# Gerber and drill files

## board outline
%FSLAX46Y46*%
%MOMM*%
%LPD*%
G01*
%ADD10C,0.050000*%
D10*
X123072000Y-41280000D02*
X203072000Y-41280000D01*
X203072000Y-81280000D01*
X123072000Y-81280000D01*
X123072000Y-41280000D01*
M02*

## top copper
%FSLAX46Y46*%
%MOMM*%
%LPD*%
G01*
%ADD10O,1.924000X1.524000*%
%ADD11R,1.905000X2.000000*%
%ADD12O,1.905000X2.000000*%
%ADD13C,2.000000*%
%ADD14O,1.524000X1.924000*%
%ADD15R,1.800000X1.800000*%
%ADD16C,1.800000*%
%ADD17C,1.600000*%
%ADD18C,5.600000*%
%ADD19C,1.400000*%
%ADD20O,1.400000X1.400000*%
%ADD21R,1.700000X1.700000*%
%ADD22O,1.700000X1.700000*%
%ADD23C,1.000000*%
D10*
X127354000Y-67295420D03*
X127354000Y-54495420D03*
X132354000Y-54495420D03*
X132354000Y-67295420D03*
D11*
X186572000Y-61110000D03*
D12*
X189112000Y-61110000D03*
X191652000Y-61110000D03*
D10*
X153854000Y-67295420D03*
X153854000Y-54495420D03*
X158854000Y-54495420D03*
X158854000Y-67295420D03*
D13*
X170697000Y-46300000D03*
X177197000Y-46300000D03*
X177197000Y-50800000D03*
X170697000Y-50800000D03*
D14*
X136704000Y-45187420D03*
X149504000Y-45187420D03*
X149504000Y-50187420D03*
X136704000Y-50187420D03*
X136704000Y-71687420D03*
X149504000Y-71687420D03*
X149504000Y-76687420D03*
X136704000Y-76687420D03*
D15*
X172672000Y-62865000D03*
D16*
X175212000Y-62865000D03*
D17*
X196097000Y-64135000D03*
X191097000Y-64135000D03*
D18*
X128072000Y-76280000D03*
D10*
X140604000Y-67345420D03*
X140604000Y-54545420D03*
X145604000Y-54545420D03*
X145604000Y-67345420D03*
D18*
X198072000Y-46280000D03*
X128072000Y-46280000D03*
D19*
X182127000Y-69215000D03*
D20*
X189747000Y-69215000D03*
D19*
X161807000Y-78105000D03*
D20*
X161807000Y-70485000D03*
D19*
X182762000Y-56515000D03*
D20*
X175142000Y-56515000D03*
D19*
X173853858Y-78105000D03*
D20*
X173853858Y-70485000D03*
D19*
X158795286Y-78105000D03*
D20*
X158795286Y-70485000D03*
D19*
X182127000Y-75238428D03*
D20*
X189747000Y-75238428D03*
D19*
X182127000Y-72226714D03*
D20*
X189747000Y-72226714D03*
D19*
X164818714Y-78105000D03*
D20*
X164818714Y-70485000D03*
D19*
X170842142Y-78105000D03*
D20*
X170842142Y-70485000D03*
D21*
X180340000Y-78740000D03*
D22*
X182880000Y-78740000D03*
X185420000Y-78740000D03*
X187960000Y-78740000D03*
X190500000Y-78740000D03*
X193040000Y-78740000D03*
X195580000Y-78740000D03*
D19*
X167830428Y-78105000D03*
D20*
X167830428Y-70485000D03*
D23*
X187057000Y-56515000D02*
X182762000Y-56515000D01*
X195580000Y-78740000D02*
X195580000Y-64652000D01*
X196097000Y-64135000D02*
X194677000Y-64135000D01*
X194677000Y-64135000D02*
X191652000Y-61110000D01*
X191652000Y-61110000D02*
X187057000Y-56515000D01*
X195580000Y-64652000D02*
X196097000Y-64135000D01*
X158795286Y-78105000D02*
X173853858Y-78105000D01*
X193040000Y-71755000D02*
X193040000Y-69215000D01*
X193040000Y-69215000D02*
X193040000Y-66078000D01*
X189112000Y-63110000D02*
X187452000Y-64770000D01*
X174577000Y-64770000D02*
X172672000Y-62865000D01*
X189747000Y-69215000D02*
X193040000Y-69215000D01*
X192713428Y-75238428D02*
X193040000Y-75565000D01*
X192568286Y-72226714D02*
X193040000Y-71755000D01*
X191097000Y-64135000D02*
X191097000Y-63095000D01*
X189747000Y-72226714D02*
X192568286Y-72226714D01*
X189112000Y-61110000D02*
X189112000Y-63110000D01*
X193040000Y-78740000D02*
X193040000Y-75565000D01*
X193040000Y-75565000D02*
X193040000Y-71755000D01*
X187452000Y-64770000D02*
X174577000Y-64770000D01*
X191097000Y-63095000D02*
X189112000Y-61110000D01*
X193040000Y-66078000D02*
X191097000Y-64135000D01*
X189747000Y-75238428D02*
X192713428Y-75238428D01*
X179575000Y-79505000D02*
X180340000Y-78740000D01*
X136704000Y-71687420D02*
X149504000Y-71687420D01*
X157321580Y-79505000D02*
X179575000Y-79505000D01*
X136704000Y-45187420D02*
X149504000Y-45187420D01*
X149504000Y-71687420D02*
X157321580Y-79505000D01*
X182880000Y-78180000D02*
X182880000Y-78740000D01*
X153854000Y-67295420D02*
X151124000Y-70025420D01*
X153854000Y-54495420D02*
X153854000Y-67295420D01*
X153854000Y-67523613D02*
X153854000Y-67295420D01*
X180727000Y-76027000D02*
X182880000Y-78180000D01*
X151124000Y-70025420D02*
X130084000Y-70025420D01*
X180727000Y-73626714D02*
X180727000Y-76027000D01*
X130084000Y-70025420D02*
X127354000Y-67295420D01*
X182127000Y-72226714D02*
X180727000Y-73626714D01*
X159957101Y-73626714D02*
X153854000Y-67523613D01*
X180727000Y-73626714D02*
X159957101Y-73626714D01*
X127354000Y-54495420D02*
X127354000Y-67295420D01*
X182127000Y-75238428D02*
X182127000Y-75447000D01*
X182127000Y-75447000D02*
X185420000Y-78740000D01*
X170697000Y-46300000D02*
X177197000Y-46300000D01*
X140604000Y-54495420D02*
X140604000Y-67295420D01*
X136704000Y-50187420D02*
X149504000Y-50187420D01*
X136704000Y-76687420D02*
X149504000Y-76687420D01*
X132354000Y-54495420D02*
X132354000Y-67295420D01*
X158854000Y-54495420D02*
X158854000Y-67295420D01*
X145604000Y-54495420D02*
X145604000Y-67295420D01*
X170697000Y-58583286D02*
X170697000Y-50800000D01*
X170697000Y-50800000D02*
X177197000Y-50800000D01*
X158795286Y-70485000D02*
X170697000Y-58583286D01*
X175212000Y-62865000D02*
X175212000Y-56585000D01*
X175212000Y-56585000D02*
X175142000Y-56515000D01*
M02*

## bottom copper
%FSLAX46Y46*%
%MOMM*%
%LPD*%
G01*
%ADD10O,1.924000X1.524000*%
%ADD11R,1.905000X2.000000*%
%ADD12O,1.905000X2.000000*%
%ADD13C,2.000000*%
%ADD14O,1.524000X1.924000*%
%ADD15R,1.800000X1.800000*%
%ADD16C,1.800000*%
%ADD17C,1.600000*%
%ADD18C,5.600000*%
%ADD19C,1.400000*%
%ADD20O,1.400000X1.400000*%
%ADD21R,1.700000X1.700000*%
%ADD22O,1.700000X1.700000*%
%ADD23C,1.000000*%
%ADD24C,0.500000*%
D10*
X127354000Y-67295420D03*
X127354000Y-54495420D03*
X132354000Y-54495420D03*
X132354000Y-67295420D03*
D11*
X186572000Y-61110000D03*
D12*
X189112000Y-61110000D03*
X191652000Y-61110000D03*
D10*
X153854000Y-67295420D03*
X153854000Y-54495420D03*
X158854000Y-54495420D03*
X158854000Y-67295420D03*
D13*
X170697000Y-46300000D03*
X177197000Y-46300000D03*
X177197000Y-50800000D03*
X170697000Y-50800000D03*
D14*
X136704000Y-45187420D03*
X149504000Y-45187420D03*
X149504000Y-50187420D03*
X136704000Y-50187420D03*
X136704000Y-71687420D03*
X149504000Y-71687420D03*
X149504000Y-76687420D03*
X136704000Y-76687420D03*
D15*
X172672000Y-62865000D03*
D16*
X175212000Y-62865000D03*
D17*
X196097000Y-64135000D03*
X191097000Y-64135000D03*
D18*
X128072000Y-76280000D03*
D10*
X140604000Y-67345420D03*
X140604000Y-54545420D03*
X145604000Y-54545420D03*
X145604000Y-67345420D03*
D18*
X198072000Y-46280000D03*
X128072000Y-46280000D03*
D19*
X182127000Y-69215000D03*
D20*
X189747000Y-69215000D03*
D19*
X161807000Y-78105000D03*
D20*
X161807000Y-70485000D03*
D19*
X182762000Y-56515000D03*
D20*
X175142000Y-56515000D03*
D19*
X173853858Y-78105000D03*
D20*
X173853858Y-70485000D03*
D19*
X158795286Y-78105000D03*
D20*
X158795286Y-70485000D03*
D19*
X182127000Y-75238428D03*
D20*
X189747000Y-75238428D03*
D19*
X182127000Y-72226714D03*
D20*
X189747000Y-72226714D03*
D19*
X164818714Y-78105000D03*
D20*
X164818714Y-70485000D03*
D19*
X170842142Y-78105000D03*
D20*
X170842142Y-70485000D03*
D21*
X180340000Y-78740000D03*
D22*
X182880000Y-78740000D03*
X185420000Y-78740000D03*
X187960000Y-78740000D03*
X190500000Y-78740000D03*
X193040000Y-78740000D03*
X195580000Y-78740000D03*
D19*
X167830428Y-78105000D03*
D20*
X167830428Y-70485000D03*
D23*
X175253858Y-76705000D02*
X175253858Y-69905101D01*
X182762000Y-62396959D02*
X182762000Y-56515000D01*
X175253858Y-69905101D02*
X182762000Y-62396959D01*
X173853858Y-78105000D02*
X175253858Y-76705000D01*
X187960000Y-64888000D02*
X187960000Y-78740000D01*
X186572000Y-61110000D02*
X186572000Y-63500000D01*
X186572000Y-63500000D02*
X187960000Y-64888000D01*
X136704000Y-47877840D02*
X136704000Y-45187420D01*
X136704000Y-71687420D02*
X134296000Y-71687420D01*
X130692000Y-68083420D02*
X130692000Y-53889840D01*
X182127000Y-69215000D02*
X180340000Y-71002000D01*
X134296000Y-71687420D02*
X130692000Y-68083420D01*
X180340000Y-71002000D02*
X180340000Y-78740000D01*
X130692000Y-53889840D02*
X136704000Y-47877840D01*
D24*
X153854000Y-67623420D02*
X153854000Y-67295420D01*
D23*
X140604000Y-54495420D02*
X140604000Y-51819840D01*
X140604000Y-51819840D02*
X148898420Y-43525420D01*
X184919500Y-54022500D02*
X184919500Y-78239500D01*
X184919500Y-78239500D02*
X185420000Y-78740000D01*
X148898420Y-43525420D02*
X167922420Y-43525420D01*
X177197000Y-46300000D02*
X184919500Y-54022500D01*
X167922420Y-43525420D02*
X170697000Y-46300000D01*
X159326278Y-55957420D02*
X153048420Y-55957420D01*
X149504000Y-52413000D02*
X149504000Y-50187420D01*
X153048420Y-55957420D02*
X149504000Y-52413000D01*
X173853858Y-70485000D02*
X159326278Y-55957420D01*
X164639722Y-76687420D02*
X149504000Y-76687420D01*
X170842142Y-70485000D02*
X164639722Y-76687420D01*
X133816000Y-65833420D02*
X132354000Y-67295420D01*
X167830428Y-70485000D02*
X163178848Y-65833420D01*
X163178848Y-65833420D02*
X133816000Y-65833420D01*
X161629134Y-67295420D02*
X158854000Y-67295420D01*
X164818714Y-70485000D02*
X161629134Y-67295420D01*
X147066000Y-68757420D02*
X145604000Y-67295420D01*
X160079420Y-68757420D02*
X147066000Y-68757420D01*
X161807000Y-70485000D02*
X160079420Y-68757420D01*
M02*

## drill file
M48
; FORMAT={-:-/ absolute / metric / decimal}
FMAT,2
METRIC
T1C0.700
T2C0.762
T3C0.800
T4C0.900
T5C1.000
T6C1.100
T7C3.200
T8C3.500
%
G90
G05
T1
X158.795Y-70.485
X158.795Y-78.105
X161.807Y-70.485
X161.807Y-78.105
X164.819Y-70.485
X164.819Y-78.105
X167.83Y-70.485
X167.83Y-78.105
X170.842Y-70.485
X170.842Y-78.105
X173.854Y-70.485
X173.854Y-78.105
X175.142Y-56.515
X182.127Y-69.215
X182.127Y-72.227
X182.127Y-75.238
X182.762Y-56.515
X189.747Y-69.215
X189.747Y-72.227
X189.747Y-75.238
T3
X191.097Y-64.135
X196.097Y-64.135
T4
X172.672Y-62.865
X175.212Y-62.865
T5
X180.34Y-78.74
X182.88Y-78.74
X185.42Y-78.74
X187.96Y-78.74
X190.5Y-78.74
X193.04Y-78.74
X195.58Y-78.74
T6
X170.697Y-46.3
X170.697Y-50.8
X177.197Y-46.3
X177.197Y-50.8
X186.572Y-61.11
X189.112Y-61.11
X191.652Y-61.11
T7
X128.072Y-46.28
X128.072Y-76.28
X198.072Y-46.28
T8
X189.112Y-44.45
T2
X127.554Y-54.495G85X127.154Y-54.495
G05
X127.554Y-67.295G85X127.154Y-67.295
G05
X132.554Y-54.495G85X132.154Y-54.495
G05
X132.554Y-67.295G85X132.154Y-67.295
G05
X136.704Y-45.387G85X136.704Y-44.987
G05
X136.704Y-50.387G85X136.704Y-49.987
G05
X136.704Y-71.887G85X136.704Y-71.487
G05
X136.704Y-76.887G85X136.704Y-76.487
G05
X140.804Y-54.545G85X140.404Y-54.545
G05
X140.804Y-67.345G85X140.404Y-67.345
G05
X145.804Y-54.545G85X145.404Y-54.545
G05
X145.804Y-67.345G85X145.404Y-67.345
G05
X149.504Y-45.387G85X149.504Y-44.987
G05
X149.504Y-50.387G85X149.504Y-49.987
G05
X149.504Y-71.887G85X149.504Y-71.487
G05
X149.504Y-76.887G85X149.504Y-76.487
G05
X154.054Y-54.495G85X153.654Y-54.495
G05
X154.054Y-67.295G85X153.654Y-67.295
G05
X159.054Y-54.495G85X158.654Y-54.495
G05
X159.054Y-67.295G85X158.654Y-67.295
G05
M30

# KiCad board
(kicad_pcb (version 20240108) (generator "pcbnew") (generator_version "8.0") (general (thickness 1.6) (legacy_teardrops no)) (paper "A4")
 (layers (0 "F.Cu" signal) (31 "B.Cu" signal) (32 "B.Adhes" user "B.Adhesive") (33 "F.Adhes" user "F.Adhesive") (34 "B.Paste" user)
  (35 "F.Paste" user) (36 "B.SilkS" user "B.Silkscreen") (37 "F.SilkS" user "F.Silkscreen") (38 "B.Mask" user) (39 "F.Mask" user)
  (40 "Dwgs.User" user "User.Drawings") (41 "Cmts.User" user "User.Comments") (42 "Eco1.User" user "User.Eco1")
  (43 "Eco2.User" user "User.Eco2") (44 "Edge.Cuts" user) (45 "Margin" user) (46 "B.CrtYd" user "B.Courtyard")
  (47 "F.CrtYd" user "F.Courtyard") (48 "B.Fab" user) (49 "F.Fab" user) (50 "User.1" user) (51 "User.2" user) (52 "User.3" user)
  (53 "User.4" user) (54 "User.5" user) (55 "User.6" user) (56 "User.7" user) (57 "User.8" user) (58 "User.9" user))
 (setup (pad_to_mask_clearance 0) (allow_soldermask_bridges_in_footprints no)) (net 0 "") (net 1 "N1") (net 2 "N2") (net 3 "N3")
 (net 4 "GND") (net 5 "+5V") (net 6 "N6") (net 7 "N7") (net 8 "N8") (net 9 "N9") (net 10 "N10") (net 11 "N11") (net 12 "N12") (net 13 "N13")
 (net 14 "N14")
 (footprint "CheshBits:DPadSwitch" (layer "F.Cu") (at 129.854 60.89542 90)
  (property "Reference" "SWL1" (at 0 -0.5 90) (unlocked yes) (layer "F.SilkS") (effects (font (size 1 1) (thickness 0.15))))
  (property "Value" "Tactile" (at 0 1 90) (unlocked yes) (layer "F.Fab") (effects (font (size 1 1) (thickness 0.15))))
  (pad "1" thru_hole oval (at -6.4 -2.5 270) (size 1.524 1.924) (drill oval 0.762 1.162) (layers "*.Cu" "*.Mask") (remove_unused_layers no)
   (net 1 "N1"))
  (pad "2" thru_hole oval (at 6.4 -2.5 270) (size 1.524 1.924) (drill oval 0.762 1.162) (layers "*.Cu" "*.Mask") (remove_unused_layers no)
   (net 1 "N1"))
  (pad "3" thru_hole oval (at 6.4 2.5 270) (size 1.524 1.924) (drill oval 0.762 1.162) (layers "*.Cu" "*.Mask") (remove_unused_layers no)
   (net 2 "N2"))
  (pad "4" thru_hole oval (at -6.4 2.5 270) (size 1.524 1.924) (drill oval 0.762 1.162) (layers "*.Cu" "*.Mask") (remove_unused_layers no)
   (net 2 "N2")))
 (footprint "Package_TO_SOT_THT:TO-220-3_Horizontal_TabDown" (layer "F.Cu") (at 186.572 61.11)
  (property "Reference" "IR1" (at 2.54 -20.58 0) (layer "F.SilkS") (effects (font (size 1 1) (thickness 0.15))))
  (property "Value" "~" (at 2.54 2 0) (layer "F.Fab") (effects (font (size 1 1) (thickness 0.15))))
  (pad "" np_thru_hole circle (at 2.54 -16.66) (size 3.5 3.5) (drill 3.5) (layers "*.Cu" "*.Mask"))
  (pad "1" thru_hole rect (at 0 0) (size 1.905 2) (drill 1.1) (layers "*.Cu" "*.Mask") (remove_unused_layers no) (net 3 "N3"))
  (pad "2" thru_hole oval (at 2.54 0) (size 1.905 2) (drill 1.1) (layers "*.Cu" "*.Mask") (remove_unused_layers no) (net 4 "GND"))
  (pad "3" thru_hole oval (at 5.08 0) (size 1.905 2) (drill 1.1) (layers "*.Cu" "*.Mask") (remove_unused_layers no) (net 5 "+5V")))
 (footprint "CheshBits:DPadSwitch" (layer "F.Cu") (at 156.354 60.89542 90)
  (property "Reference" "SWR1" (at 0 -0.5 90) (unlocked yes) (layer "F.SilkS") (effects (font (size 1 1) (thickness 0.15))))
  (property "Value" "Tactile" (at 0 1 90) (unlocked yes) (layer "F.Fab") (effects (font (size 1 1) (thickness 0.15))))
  (pad "1" thru_hole oval (at -6.4 -2.5 270) (size 1.524 1.924) (drill oval 0.762 1.162) (layers "*.Cu" "*.Mask") (remove_unused_layers no)
   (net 1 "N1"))
  (pad "2" thru_hole oval (at 6.4 -2.5 270) (size 1.524 1.924) (drill oval 0.762 1.162) (layers "*.Cu" "*.Mask") (remove_unused_layers no)
   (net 1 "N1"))
  (pad "3" thru_hole oval (at 6.4 2.5 270) (size 1.524 1.924) (drill oval 0.762 1.162) (layers "*.Cu" "*.Mask") (remove_unused_layers no)
   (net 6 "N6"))
  (pad "4" thru_hole oval (at -6.4 2.5 270) (size 1.524 1.924) (drill oval 0.762 1.162) (layers "*.Cu" "*.Mask") (remove_unused_layers no)
   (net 6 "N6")))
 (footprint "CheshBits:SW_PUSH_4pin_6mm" (layer "F.Cu") (at 170.697 46.3)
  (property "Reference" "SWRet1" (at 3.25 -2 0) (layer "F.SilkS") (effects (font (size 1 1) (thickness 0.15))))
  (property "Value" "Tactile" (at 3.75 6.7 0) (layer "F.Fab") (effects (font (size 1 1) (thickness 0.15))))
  (pad "1" thru_hole circle (at 0 0 90) (size 2 2) (drill 1.1) (layers "*.Cu" "*.Mask") (remove_unused_layers no) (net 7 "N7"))
  (pad "2" thru_hole circle (at 6.5 0 90) (size 2 2) (drill 1.1) (layers "*.Cu" "*.Mask") (remove_unused_layers no) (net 7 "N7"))
  (pad "3" thru_hole circle (at 6.5 4.5 90) (size 2 2) (drill 1.1) (layers "*.Cu" "*.Mask") (remove_unused_layers no) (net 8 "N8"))
  (pad "4" thru_hole circle (at 0 4.5 90) (size 2 2) (drill 1.1) (layers "*.Cu" "*.Mask") (remove_unused_layers no) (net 8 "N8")))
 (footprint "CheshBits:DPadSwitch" (layer "F.Cu") (at 143.104 47.68742)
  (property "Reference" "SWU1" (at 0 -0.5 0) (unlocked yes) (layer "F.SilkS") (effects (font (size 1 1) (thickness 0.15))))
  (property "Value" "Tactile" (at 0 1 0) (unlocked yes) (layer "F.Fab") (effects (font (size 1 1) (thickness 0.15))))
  (pad "1" thru_hole oval (at -6.4 -2.5 180) (size 1.524 1.924) (drill oval 0.762 1.162) (layers "*.Cu" "*.Mask") (remove_unused_layers no)
   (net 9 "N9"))
  (pad "2" thru_hole oval (at 6.4 -2.5 180) (size 1.524 1.924) (drill oval 0.762 1.162) (layers "*.Cu" "*.Mask") (remove_unused_layers no)
   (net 9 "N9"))
  (pad "3" thru_hole oval (at 6.4 2.5 180) (size 1.524 1.924) (drill oval 0.762 1.162) (layers "*.Cu" "*.Mask") (remove_unused_layers no)
   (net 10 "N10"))
  (pad "4" thru_hole oval (at -6.4 2.5 180) (size 1.524 1.924) (drill oval 0.762 1.162) (layers "*.Cu" "*.Mask") (remove_unused_layers no)
   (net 10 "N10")))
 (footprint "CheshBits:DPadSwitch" (layer "F.Cu") (at 143.104 74.18742)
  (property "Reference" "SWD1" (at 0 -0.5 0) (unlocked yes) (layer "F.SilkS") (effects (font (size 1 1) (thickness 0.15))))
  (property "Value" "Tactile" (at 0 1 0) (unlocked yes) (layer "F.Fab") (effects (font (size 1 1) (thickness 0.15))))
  (pad "1" thru_hole oval (at -6.4 -2.5 180) (size 1.524 1.924) (drill oval 0.762 1.162) (layers "*.Cu" "*.Mask") (remove_unused_layers no)
   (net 9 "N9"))
  (pad "2" thru_hole oval (at 6.4 -2.5 180) (size 1.524 1.924) (drill oval 0.762 1.162) (layers "*.Cu" "*.Mask") (remove_unused_layers no)
   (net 9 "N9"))
  (pad "3" thru_hole oval (at 6.4 2.5 180) (size 1.524 1.924) (drill oval 0.762 1.162) (layers "*.Cu" "*.Mask") (remove_unused_layers no)
   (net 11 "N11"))
  (pad "4" thru_hole oval (at -6.4 2.5 180) (size 1.524 1.924) (drill oval 0.762 1.162) (layers "*.Cu" "*.Mask") (remove_unused_layers no)
   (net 11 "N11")))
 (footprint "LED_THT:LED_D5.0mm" (layer "F.Cu") (at 172.672 62.865)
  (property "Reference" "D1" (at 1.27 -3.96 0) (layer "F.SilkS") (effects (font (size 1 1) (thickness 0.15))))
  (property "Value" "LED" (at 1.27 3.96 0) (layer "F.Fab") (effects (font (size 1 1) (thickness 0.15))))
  (pad "1" thru_hole rect (at 0 0) (size 1.8 1.8) (drill 0.9) (layers "*.Cu" "*.Mask") (remove_unused_layers no) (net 4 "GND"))
  (pad "2" thru_hole circle (at 2.54 0) (size 1.8 1.8) (drill 0.9) (layers "*.Cu" "*.Mask") (remove_unused_layers no) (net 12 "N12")))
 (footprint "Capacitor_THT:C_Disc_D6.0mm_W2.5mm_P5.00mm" (layer "F.Cu") (at 196.097 64.135 180)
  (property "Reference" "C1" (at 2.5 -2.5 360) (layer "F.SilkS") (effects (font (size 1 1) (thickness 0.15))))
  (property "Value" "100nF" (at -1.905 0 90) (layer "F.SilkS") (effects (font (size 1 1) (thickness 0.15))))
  (pad "1" thru_hole circle (at 0 0 180) (size 1.6 1.6) (drill 0.8) (layers "*.Cu" "*.Mask") (remove_unused_layers no) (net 5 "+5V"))
  (pad "2" thru_hole circle (at 5 0 180) (size 1.6 1.6) (drill 0.8) (layers "*.Cu" "*.Mask") (remove_unused_layers no) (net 4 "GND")))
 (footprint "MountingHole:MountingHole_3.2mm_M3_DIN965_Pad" (layer "F.Cu") (at 128.072 76.28)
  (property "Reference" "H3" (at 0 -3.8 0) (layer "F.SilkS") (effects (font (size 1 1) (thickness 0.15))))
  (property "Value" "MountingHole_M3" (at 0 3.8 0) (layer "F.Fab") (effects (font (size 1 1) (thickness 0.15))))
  (pad "1" thru_hole circle (at 0 0) (size 5.6 5.6) (drill 3.2) (layers "*.Cu" "*.Mask") (remove_unused_layers no)))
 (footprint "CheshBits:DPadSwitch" (layer "F.Cu") (at 143.104 60.94542 90)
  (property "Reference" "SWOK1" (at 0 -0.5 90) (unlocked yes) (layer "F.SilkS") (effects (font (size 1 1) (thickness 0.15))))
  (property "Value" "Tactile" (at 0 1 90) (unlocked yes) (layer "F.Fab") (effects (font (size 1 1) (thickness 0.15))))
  (pad "1" thru_hole oval (at -6.4 -2.5 270) (size 1.524 1.924) (drill oval 0.762 1.162) (layers "*.Cu" "*.Mask") (remove_unused_layers no)
   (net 7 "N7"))
  (pad "2" thru_hole oval (at 6.4 -2.5 270) (size 1.524 1.924) (drill oval 0.762 1.162) (layers "*.Cu" "*.Mask") (remove_unused_layers no)
   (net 7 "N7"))
  (pad "3" thru_hole oval (at 6.4 2.5 270) (size 1.524 1.924) (drill oval 0.762 1.162) (layers "*.Cu" "*.Mask") (remove_unused_layers no)
   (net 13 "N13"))
  (pad "4" thru_hole oval (at -6.4 2.5 270) (size 1.524 1.924) (drill oval 0.762 1.162) (layers "*.Cu" "*.Mask") (remove_unused_layers no)
   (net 13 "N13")))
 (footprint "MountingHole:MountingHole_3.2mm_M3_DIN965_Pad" (layer "F.Cu") (at 198.072 46.28)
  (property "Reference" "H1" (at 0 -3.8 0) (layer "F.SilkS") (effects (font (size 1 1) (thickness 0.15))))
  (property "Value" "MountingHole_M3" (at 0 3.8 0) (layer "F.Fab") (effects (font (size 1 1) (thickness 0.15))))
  (pad "1" thru_hole circle (at 0 0) (size 5.6 5.6) (drill 3.2) (layers "*.Cu" "*.Mask") (remove_unused_layers no)))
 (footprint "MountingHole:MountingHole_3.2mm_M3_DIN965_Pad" (layer "F.Cu") (at 128.072 46.28)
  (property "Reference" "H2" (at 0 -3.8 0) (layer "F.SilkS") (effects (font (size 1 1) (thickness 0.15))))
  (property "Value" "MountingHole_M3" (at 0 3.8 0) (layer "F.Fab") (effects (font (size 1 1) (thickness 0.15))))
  (pad "1" thru_hole circle (at 0 0) (size 5.6 5.6) (drill 3.2) (layers "*.Cu" "*.Mask") (remove_unused_layers no)))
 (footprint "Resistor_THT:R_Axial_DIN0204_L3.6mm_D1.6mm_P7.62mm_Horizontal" (layer "B.Cu") (at 182.127 69.215)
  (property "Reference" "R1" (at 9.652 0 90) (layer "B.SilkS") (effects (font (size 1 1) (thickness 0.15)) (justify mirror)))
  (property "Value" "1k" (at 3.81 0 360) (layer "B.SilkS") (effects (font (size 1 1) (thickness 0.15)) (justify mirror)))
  (pad "1" thru_hole circle (at 0 0) (size 1.4 1.4) (drill 0.7) (layers "*.Cu" "*.Mask") (remove_unused_layers no) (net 9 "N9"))
  (pad "2" thru_hole oval (at 7.62 0) (size 1.4 1.4) (drill 0.7) (layers "*.Cu" "*.Mask") (remove_unused_layers no) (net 4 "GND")))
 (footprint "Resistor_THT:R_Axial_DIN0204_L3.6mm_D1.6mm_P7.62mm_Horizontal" (layer "B.Cu") (at 161.807 78.105 90)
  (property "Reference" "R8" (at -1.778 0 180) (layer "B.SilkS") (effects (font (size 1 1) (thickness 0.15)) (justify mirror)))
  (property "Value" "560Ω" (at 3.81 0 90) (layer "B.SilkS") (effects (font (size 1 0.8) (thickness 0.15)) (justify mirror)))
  (pad "1" thru_hole circle (at 0 0 90) (size 1.4 1.4) (drill 0.7) (layers "*.Cu" "*.Mask") (remove_unused_layers no) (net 5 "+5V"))
  (pad "2" thru_hole oval (at 7.62 0 90) (size 1.4 1.4) (drill 0.7) (layers "*.Cu" "*.Mask") (remove_unused_layers no) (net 13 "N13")))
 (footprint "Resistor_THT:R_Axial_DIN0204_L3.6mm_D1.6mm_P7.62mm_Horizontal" (layer "B.Cu") (at 182.762 56.515 180)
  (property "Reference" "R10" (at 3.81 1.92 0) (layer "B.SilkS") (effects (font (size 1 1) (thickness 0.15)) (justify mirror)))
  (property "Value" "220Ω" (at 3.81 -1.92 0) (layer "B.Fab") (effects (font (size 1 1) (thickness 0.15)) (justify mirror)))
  (pad "1" thru_hole circle (at 0 0 180) (size 1.4 1.4) (drill 0.7) (layers "*.Cu" "*.Mask") (remove_unused_layers no) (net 5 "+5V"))
  (pad "2" thru_hole oval (at 7.62 0 180) (size 1.4 1.4) (drill 0.7) (layers "*.Cu" "*.Mask") (remove_unused_layers no) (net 12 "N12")))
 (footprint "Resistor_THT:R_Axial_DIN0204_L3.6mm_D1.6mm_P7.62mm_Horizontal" (layer "B.Cu") (at 173.853858 78.105 90)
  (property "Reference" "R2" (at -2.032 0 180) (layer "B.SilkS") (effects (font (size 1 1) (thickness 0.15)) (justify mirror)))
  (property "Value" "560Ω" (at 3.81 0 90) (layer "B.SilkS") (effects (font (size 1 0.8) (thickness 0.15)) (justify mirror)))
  (pad "1" thru_hole circle (at 0 0 90) (size 1.4 1.4) (drill 0.7) (layers "*.Cu" "*.Mask") (remove_unused_layers no) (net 5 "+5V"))
  (pad "2" thru_hole oval (at 7.62 0 90) (size 1.4 1.4) (drill 0.7) (layers "*.Cu" "*.Mask") (remove_unused_layers no) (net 10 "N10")))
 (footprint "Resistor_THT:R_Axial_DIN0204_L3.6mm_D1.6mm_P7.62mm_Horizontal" (layer "B.Cu") (at 158.795286 78.105 90)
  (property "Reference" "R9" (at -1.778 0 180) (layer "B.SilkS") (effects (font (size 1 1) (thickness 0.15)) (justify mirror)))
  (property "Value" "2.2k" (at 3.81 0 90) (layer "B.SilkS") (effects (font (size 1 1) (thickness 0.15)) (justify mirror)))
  (pad "1" thru_hole circle (at 0 0 90) (size 1.4 1.4) (drill 0.7) (layers "*.Cu" "*.Mask") (remove_unused_layers no) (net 5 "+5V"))
  (pad "2" thru_hole oval (at 7.62 0 90) (size 1.4 1.4) (drill 0.7) (layers "*.Cu" "*.Mask") (remove_unused_layers no) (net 8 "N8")))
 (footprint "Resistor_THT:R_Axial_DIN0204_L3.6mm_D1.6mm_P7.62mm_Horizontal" (layer "B.Cu") (at 182.127 75.238428)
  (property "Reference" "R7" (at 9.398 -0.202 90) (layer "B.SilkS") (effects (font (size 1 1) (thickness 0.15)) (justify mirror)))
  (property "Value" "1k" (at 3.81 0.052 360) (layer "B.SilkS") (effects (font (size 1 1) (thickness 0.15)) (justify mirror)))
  (pad "1" thru_hole circle (at 0 0) (size 1.4 1.4) (drill 0.7) (layers "*.Cu" "*.Mask") (remove_unused_layers no) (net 7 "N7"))
  (pad "2" thru_hole oval (at 7.62 0) (size 1.4 1.4) (drill 0.7) (layers "*.Cu" "*.Mask") (remove_unused_layers no) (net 4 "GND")))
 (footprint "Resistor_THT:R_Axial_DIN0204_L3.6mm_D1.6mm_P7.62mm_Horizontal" (layer "B.Cu") (at 182.127 72.226714)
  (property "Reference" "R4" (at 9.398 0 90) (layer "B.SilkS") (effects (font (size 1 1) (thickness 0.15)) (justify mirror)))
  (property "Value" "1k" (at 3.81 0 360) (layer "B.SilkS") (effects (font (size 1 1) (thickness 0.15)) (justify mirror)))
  (pad "1" thru_hole circle (at 0 0) (size 1.4 1.4) (drill 0.7) (layers "*.Cu" "*.Mask") (remove_unused_layers no) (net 1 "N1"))
  (pad "2" thru_hole oval (at 7.62 0) (size 1.4 1.4) (drill 0.7) (layers "*.Cu" "*.Mask") (remove_unused_layers no) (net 4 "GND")))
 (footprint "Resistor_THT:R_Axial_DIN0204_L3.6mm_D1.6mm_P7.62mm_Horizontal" (layer "B.Cu") (at 164.818714 78.105 90)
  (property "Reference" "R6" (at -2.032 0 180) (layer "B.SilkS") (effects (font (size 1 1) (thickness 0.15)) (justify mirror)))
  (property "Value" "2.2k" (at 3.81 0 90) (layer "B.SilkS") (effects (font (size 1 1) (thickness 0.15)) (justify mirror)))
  (pad "1" thru_hole circle (at 0 0 90) (size 1.4 1.4) (drill 0.7) (layers "*.Cu" "*.Mask") (remove_unused_layers no) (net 5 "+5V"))
  (pad "2" thru_hole oval (at 7.62 0 90) (size 1.4 1.4) (drill 0.7) (layers "*.Cu" "*.Mask") (remove_unused_layers no) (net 6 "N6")))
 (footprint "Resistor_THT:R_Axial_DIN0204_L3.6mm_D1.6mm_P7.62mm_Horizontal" (layer "B.Cu") (at 170.842142 78.105 90)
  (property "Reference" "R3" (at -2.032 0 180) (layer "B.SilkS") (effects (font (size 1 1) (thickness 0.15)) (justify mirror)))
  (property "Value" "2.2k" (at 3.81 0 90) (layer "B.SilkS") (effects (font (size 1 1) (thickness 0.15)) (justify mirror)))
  (pad "1" thru_hole circle (at 0 0 90) (size 1.4 1.4) (drill 0.7) (layers "*.Cu" "*.Mask") (remove_unused_layers no) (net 5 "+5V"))
  (pad "2" thru_hole oval (at 7.62 0 90) (size 1.4 1.4) (drill 0.7) (layers "*.Cu" "*.Mask") (remove_unused_layers no) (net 11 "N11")))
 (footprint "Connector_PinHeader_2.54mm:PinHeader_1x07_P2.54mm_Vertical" (layer "B.Cu") (at 180.34 78.74 -90)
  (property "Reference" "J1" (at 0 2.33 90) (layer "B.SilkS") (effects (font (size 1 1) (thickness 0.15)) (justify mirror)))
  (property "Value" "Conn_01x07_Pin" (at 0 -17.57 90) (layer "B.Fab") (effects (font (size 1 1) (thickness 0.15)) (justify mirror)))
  (pad "1" thru_hole rect (at 0 0 270) (size 1.7 1.7) (drill 1) (layers "*.Cu" "*.Mask") (remove_unused_layers no) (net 9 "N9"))
  (pad "2" thru_hole oval (at 0 -2.54 270) (size 1.7 1.7) (drill 1) (layers "*.Cu" "*.Mask") (remove_unused_layers no) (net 1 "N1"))
  (pad "3" thru_hole oval (at 0 -5.08 270) (size 1.7 1.7) (drill 1) (layers "*.Cu" "*.Mask") (remove_unused_layers no) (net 7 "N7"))
  (pad "4" thru_hole oval (at 0 -7.62 270) (size 1.7 1.7) (drill 1) (layers "*.Cu" "*.Mask") (remove_unused_layers no) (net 3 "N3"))
  (pad "5" thru_hole oval (at 0 -10.16 270) (size 1.7 1.7) (drill 1) (layers "*.Cu" "*.Mask") (remove_unused_layers no) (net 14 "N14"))
  (pad "6" thru_hole oval (at 0 -12.7 270) (size 1.7 1.7) (drill 1) (layers "*.Cu" "*.Mask") (remove_unused_layers no) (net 4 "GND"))
  (pad "7" thru_hole oval (at 0 -15.24 270) (size 1.7 1.7) (drill 1) (layers "*.Cu" "*.Mask") (remove_unused_layers no) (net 5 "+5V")))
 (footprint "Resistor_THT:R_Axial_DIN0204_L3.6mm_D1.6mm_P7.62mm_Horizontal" (layer "B.Cu") (at 167.830428 78.105 90)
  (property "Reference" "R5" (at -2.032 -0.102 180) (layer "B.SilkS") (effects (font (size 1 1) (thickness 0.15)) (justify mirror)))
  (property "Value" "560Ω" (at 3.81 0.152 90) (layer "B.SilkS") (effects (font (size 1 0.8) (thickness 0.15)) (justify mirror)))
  (pad "1" thru_hole circle (at 0 0 90) (size 1.4 1.4) (drill 0.7) (layers "*.Cu" "*.Mask") (remove_unused_layers no) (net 5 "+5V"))
  (pad "2" thru_hole oval (at 7.62 0 90) (size 1.4 1.4) (drill 0.7) (layers "*.Cu" "*.Mask") (remove_unused_layers no) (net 2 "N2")))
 (gr_rect (start 123.072 41.28) (end 203.072 81.28) (stroke (width 0.05) (type default)) (fill none) (layer "Edge.Cuts"))
 (segment (start 187.057 56.515) (end 182.762 56.515) (width 1) (layer "F.Cu") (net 5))
 (segment (start 195.58 78.74) (end 195.58 64.652) (width 1) (layer "F.Cu") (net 5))
 (segment (start 196.097 64.135) (end 194.677 64.135) (width 1) (layer "F.Cu") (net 5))
 (segment (start 194.677 64.135) (end 191.652 61.11) (width 1) (layer "F.Cu") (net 5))
 (segment (start 191.652 61.11) (end 187.057 56.515) (width 1) (layer "F.Cu") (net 5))
 (segment (start 195.58 64.652) (end 196.097 64.135) (width 1) (layer "F.Cu") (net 5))
 (segment (start 158.795286 78.105) (end 173.853858 78.105) (width 1) (layer "F.Cu") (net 5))
 (segment (start 175.253858 76.705) (end 175.253858 69.905101) (width 1) (layer "B.Cu") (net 5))
 (segment (start 182.762 62.396959) (end 182.762 56.515) (width 1) (layer "B.Cu") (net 5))
 (segment (start 175.253858 69.905101) (end 182.762 62.396959) (width 1) (layer "B.Cu") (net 5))
 (segment (start 173.853858 78.105) (end 175.253858 76.705) (width 1) (layer "B.Cu") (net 5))
 (segment (start 193.04 71.755) (end 193.04 69.215) (width 1) (layer "F.Cu") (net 4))
 (segment (start 193.04 69.215) (end 193.04 66.078) (width 1) (layer "F.Cu") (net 4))
 (segment (start 189.112 63.11) (end 187.452 64.77) (width 1) (layer "F.Cu") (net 4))
 (segment (start 174.577 64.77) (end 172.672 62.865) (width 1) (layer "F.Cu") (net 4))
 (segment (start 189.747 69.215) (end 193.04 69.215) (width 1) (layer "F.Cu") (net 4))
 (segment (start 192.713428 75.238428) (end 193.04 75.565) (width 1) (layer "F.Cu") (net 4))
 (segment (start 192.568286 72.226714) (end 193.04 71.755) (width 1) (layer "F.Cu") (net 4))
 (segment (start 191.097 64.135) (end 191.097 63.095) (width 1) (layer "F.Cu") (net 4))
 (segment (start 189.747 72.226714) (end 192.568286 72.226714) (width 1) (layer "F.Cu") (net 4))
 (segment (start 189.112 61.11) (end 189.112 63.11) (width 1) (layer "F.Cu") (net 4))
 (segment (start 193.04 78.74) (end 193.04 75.565) (width 1) (layer "F.Cu") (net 4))
 (segment (start 193.04 75.565) (end 193.04 71.755) (width 1) (layer "F.Cu") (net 4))
 (segment (start 187.452 64.77) (end 174.577 64.77) (width 1) (layer "F.Cu") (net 4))
 (segment (start 191.097 63.095) (end 189.112 61.11) (width 1) (layer "F.Cu") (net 4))
 (segment (start 193.04 66.078) (end 191.097 64.135) (width 1) (layer "F.Cu") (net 4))
 (segment (start 189.747 75.238428) (end 192.713428 75.238428) (width 1) (layer "F.Cu") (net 4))
 (segment (start 187.96 64.888) (end 187.96 78.74) (width 1) (layer "B.Cu") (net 3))
 (segment (start 186.572 61.11) (end 186.572 63.5) (width 1) (layer "B.Cu") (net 3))
 (segment (start 186.572 63.5) (end 187.96 64.888) (width 1) (layer "B.Cu") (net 3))
 (segment (start 179.575 79.505) (end 180.34 78.74) (width 1) (layer "F.Cu") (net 9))
 (segment (start 136.704 71.68742) (end 149.504 71.68742) (width 1) (layer "F.Cu") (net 9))
 (segment (start 157.32158 79.505) (end 179.575 79.505) (width 1) (layer "F.Cu") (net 9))
 (segment (start 136.704 45.18742) (end 149.504 45.18742) (width 1) (layer "F.Cu") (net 9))
 (segment (start 149.504 71.68742) (end 157.32158 79.505) (width 1) (layer "F.Cu") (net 9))
 (segment (start 136.704 47.87784) (end 136.704 45.18742) (width 1) (layer "B.Cu") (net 9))
 (segment (start 136.704 71.68742) (end 134.296 71.68742) (width 1) (layer "B.Cu") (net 9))
 (segment (start 130.692 68.08342) (end 130.692 53.88984) (width 1) (layer "B.Cu") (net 9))
 (segment (start 182.127 69.215) (end 180.34 71.002) (width 1) (layer "B.Cu") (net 9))
 (segment (start 134.296 71.68742) (end 130.692 68.08342) (width 1) (layer "B.Cu") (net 9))
 (segment (start 180.34 71.002) (end 180.34 78.74) (width 1) (layer "B.Cu") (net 9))
 (segment (start 130.692 53.88984) (end 136.704 47.87784) (width 1) (layer "B.Cu") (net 9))
 (segment (start 182.88 78.18) (end 182.88 78.74) (width 1) (layer "F.Cu") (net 1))
 (segment (start 153.854 67.29542) (end 151.124 70.02542) (width 1) (layer "F.Cu") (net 1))
 (segment (start 153.854 54.49542) (end 153.854 67.29542) (width 1) (layer "F.Cu") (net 1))
 (segment (start 153.854 67.523613) (end 153.854 67.29542) (width 1) (layer "F.Cu") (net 1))
 (segment (start 180.727 76.027) (end 182.88 78.18) (width 1) (layer "F.Cu") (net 1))
 (segment (start 151.124 70.02542) (end 130.084 70.02542) (width 1) (layer "F.Cu") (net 1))
 (segment (start 180.727 73.626714) (end 180.727 76.027) (width 1) (layer "F.Cu") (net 1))
 (segment (start 130.084 70.02542) (end 127.354 67.29542) (width 1) (layer "F.Cu") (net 1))
 (segment (start 182.127 72.226714) (end 180.727 73.626714) (width 1) (layer "F.Cu") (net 1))
 (segment (start 159.957101 73.626714) (end 153.854 67.523613) (width 1) (layer "F.Cu") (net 1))
 (segment (start 180.727 73.626714) (end 159.957101 73.626714) (width 1) (layer "F.Cu") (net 1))
 (segment (start 127.354 54.49542) (end 127.354 67.29542) (width 1) (layer "F.Cu") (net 1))
 (segment (start 153.854 67.62342) (end 153.854 67.29542) (width 0.5) (layer "B.Cu") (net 1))
 (segment (start 182.127 75.238428) (end 182.127 75.447) (width 1) (layer "F.Cu") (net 7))
 (segment (start 182.127 75.447) (end 185.42 78.74) (width 1) (layer "F.Cu") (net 7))
 (segment (start 170.697 46.3) (end 177.197 46.3) (width 1) (layer "F.Cu") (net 7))
 (segment (start 140.604 54.49542) (end 140.604 67.29542) (width 1) (layer "F.Cu") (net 7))
 (segment (start 140.604 54.49542) (end 140.604 51.81984) (width 1) (layer "B.Cu") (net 7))
 (segment (start 140.604 51.81984) (end 148.89842 43.52542) (width 1) (layer "B.Cu") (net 7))
 (segment (start 184.9195 54.0225) (end 184.9195 78.2395) (width 1) (layer "B.Cu") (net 7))
 (segment (start 184.9195 78.2395) (end 185.42 78.74) (width 1) (layer "B.Cu") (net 7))
 (segment (start 148.89842 43.52542) (end 167.92242 43.52542) (width 1) (layer "B.Cu") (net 7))
 (segment (start 177.197 46.3) (end 184.9195 54.0225) (width 1) (layer "B.Cu") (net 7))
 (segment (start 167.92242 43.52542) (end 170.697 46.3) (width 1) (layer "B.Cu") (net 7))
 (segment (start 136.704 50.18742) (end 149.504 50.18742) (width 1) (layer "F.Cu") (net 10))
 (segment (start 159.326278 55.95742) (end 153.04842 55.95742) (width 1) (layer "B.Cu") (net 10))
 (segment (start 149.504 52.413) (end 149.504 50.18742) (width 1) (layer "B.Cu") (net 10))
 (segment (start 153.04842 55.95742) (end 149.504 52.413) (width 1) (layer "B.Cu") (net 10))
 (segment (start 173.853858 70.485) (end 159.326278 55.95742) (width 1) (layer "B.Cu") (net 10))
 (segment (start 136.704 76.68742) (end 149.504 76.68742) (width 1) (layer "F.Cu") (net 11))
 (segment (start 164.639722 76.68742) (end 149.504 76.68742) (width 1) (layer "B.Cu") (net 11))
 (segment (start 170.842142 70.485) (end 164.639722 76.68742) (width 1) (layer "B.Cu") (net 11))
 (segment (start 132.354 54.49542) (end 132.354 67.29542) (width 1) (layer "F.Cu") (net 2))
 (segment (start 133.816 65.83342) (end 132.354 67.29542) (width 1) (layer "B.Cu") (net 2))
 (segment (start 167.830428 70.485) (end 163.178848 65.83342) (width 1) (layer "B.Cu") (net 2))
 (segment (start 163.178848 65.83342) (end 133.816 65.83342) (width 1) (layer "B.Cu") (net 2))
 (segment (start 158.854 54.49542) (end 158.854 67.29542) (width 1) (layer "F.Cu") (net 6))
 (segment (start 161.629134 67.29542) (end 158.854 67.29542) (width 1) (layer "B.Cu") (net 6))
 (segment (start 164.818714 70.485) (end 161.629134 67.29542) (width 1) (layer "B.Cu") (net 6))
 (segment (start 145.604 54.49542) (end 145.604 67.29542) (width 1) (layer "F.Cu") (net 13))
 (segment (start 147.066 68.75742) (end 145.604 67.29542) (width 1) (layer "B.Cu") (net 13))
 (segment (start 160.07942 68.75742) (end 147.066 68.75742) (width 1) (layer "B.Cu") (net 13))
 (segment (start 161.807 70.485) (end 160.07942 68.75742) (width 1) (layer "B.Cu") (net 13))
 (segment (start 170.697 58.583286) (end 170.697 50.8) (width 1) (layer "F.Cu") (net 8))
 (segment (start 170.697 50.8) (end 177.197 50.8) (width 1) (layer "F.Cu") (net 8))
 (segment (start 158.795286 70.485) (end 170.697 58.583286) (width 1) (layer "F.Cu") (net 8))
 (segment (start 175.212 62.865) (end 175.212 56.585) (width 1) (layer "F.Cu") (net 12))
 (segment (start 175.212 56.585) (end 175.142 56.515) (width 1) (layer "F.Cu") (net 12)))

